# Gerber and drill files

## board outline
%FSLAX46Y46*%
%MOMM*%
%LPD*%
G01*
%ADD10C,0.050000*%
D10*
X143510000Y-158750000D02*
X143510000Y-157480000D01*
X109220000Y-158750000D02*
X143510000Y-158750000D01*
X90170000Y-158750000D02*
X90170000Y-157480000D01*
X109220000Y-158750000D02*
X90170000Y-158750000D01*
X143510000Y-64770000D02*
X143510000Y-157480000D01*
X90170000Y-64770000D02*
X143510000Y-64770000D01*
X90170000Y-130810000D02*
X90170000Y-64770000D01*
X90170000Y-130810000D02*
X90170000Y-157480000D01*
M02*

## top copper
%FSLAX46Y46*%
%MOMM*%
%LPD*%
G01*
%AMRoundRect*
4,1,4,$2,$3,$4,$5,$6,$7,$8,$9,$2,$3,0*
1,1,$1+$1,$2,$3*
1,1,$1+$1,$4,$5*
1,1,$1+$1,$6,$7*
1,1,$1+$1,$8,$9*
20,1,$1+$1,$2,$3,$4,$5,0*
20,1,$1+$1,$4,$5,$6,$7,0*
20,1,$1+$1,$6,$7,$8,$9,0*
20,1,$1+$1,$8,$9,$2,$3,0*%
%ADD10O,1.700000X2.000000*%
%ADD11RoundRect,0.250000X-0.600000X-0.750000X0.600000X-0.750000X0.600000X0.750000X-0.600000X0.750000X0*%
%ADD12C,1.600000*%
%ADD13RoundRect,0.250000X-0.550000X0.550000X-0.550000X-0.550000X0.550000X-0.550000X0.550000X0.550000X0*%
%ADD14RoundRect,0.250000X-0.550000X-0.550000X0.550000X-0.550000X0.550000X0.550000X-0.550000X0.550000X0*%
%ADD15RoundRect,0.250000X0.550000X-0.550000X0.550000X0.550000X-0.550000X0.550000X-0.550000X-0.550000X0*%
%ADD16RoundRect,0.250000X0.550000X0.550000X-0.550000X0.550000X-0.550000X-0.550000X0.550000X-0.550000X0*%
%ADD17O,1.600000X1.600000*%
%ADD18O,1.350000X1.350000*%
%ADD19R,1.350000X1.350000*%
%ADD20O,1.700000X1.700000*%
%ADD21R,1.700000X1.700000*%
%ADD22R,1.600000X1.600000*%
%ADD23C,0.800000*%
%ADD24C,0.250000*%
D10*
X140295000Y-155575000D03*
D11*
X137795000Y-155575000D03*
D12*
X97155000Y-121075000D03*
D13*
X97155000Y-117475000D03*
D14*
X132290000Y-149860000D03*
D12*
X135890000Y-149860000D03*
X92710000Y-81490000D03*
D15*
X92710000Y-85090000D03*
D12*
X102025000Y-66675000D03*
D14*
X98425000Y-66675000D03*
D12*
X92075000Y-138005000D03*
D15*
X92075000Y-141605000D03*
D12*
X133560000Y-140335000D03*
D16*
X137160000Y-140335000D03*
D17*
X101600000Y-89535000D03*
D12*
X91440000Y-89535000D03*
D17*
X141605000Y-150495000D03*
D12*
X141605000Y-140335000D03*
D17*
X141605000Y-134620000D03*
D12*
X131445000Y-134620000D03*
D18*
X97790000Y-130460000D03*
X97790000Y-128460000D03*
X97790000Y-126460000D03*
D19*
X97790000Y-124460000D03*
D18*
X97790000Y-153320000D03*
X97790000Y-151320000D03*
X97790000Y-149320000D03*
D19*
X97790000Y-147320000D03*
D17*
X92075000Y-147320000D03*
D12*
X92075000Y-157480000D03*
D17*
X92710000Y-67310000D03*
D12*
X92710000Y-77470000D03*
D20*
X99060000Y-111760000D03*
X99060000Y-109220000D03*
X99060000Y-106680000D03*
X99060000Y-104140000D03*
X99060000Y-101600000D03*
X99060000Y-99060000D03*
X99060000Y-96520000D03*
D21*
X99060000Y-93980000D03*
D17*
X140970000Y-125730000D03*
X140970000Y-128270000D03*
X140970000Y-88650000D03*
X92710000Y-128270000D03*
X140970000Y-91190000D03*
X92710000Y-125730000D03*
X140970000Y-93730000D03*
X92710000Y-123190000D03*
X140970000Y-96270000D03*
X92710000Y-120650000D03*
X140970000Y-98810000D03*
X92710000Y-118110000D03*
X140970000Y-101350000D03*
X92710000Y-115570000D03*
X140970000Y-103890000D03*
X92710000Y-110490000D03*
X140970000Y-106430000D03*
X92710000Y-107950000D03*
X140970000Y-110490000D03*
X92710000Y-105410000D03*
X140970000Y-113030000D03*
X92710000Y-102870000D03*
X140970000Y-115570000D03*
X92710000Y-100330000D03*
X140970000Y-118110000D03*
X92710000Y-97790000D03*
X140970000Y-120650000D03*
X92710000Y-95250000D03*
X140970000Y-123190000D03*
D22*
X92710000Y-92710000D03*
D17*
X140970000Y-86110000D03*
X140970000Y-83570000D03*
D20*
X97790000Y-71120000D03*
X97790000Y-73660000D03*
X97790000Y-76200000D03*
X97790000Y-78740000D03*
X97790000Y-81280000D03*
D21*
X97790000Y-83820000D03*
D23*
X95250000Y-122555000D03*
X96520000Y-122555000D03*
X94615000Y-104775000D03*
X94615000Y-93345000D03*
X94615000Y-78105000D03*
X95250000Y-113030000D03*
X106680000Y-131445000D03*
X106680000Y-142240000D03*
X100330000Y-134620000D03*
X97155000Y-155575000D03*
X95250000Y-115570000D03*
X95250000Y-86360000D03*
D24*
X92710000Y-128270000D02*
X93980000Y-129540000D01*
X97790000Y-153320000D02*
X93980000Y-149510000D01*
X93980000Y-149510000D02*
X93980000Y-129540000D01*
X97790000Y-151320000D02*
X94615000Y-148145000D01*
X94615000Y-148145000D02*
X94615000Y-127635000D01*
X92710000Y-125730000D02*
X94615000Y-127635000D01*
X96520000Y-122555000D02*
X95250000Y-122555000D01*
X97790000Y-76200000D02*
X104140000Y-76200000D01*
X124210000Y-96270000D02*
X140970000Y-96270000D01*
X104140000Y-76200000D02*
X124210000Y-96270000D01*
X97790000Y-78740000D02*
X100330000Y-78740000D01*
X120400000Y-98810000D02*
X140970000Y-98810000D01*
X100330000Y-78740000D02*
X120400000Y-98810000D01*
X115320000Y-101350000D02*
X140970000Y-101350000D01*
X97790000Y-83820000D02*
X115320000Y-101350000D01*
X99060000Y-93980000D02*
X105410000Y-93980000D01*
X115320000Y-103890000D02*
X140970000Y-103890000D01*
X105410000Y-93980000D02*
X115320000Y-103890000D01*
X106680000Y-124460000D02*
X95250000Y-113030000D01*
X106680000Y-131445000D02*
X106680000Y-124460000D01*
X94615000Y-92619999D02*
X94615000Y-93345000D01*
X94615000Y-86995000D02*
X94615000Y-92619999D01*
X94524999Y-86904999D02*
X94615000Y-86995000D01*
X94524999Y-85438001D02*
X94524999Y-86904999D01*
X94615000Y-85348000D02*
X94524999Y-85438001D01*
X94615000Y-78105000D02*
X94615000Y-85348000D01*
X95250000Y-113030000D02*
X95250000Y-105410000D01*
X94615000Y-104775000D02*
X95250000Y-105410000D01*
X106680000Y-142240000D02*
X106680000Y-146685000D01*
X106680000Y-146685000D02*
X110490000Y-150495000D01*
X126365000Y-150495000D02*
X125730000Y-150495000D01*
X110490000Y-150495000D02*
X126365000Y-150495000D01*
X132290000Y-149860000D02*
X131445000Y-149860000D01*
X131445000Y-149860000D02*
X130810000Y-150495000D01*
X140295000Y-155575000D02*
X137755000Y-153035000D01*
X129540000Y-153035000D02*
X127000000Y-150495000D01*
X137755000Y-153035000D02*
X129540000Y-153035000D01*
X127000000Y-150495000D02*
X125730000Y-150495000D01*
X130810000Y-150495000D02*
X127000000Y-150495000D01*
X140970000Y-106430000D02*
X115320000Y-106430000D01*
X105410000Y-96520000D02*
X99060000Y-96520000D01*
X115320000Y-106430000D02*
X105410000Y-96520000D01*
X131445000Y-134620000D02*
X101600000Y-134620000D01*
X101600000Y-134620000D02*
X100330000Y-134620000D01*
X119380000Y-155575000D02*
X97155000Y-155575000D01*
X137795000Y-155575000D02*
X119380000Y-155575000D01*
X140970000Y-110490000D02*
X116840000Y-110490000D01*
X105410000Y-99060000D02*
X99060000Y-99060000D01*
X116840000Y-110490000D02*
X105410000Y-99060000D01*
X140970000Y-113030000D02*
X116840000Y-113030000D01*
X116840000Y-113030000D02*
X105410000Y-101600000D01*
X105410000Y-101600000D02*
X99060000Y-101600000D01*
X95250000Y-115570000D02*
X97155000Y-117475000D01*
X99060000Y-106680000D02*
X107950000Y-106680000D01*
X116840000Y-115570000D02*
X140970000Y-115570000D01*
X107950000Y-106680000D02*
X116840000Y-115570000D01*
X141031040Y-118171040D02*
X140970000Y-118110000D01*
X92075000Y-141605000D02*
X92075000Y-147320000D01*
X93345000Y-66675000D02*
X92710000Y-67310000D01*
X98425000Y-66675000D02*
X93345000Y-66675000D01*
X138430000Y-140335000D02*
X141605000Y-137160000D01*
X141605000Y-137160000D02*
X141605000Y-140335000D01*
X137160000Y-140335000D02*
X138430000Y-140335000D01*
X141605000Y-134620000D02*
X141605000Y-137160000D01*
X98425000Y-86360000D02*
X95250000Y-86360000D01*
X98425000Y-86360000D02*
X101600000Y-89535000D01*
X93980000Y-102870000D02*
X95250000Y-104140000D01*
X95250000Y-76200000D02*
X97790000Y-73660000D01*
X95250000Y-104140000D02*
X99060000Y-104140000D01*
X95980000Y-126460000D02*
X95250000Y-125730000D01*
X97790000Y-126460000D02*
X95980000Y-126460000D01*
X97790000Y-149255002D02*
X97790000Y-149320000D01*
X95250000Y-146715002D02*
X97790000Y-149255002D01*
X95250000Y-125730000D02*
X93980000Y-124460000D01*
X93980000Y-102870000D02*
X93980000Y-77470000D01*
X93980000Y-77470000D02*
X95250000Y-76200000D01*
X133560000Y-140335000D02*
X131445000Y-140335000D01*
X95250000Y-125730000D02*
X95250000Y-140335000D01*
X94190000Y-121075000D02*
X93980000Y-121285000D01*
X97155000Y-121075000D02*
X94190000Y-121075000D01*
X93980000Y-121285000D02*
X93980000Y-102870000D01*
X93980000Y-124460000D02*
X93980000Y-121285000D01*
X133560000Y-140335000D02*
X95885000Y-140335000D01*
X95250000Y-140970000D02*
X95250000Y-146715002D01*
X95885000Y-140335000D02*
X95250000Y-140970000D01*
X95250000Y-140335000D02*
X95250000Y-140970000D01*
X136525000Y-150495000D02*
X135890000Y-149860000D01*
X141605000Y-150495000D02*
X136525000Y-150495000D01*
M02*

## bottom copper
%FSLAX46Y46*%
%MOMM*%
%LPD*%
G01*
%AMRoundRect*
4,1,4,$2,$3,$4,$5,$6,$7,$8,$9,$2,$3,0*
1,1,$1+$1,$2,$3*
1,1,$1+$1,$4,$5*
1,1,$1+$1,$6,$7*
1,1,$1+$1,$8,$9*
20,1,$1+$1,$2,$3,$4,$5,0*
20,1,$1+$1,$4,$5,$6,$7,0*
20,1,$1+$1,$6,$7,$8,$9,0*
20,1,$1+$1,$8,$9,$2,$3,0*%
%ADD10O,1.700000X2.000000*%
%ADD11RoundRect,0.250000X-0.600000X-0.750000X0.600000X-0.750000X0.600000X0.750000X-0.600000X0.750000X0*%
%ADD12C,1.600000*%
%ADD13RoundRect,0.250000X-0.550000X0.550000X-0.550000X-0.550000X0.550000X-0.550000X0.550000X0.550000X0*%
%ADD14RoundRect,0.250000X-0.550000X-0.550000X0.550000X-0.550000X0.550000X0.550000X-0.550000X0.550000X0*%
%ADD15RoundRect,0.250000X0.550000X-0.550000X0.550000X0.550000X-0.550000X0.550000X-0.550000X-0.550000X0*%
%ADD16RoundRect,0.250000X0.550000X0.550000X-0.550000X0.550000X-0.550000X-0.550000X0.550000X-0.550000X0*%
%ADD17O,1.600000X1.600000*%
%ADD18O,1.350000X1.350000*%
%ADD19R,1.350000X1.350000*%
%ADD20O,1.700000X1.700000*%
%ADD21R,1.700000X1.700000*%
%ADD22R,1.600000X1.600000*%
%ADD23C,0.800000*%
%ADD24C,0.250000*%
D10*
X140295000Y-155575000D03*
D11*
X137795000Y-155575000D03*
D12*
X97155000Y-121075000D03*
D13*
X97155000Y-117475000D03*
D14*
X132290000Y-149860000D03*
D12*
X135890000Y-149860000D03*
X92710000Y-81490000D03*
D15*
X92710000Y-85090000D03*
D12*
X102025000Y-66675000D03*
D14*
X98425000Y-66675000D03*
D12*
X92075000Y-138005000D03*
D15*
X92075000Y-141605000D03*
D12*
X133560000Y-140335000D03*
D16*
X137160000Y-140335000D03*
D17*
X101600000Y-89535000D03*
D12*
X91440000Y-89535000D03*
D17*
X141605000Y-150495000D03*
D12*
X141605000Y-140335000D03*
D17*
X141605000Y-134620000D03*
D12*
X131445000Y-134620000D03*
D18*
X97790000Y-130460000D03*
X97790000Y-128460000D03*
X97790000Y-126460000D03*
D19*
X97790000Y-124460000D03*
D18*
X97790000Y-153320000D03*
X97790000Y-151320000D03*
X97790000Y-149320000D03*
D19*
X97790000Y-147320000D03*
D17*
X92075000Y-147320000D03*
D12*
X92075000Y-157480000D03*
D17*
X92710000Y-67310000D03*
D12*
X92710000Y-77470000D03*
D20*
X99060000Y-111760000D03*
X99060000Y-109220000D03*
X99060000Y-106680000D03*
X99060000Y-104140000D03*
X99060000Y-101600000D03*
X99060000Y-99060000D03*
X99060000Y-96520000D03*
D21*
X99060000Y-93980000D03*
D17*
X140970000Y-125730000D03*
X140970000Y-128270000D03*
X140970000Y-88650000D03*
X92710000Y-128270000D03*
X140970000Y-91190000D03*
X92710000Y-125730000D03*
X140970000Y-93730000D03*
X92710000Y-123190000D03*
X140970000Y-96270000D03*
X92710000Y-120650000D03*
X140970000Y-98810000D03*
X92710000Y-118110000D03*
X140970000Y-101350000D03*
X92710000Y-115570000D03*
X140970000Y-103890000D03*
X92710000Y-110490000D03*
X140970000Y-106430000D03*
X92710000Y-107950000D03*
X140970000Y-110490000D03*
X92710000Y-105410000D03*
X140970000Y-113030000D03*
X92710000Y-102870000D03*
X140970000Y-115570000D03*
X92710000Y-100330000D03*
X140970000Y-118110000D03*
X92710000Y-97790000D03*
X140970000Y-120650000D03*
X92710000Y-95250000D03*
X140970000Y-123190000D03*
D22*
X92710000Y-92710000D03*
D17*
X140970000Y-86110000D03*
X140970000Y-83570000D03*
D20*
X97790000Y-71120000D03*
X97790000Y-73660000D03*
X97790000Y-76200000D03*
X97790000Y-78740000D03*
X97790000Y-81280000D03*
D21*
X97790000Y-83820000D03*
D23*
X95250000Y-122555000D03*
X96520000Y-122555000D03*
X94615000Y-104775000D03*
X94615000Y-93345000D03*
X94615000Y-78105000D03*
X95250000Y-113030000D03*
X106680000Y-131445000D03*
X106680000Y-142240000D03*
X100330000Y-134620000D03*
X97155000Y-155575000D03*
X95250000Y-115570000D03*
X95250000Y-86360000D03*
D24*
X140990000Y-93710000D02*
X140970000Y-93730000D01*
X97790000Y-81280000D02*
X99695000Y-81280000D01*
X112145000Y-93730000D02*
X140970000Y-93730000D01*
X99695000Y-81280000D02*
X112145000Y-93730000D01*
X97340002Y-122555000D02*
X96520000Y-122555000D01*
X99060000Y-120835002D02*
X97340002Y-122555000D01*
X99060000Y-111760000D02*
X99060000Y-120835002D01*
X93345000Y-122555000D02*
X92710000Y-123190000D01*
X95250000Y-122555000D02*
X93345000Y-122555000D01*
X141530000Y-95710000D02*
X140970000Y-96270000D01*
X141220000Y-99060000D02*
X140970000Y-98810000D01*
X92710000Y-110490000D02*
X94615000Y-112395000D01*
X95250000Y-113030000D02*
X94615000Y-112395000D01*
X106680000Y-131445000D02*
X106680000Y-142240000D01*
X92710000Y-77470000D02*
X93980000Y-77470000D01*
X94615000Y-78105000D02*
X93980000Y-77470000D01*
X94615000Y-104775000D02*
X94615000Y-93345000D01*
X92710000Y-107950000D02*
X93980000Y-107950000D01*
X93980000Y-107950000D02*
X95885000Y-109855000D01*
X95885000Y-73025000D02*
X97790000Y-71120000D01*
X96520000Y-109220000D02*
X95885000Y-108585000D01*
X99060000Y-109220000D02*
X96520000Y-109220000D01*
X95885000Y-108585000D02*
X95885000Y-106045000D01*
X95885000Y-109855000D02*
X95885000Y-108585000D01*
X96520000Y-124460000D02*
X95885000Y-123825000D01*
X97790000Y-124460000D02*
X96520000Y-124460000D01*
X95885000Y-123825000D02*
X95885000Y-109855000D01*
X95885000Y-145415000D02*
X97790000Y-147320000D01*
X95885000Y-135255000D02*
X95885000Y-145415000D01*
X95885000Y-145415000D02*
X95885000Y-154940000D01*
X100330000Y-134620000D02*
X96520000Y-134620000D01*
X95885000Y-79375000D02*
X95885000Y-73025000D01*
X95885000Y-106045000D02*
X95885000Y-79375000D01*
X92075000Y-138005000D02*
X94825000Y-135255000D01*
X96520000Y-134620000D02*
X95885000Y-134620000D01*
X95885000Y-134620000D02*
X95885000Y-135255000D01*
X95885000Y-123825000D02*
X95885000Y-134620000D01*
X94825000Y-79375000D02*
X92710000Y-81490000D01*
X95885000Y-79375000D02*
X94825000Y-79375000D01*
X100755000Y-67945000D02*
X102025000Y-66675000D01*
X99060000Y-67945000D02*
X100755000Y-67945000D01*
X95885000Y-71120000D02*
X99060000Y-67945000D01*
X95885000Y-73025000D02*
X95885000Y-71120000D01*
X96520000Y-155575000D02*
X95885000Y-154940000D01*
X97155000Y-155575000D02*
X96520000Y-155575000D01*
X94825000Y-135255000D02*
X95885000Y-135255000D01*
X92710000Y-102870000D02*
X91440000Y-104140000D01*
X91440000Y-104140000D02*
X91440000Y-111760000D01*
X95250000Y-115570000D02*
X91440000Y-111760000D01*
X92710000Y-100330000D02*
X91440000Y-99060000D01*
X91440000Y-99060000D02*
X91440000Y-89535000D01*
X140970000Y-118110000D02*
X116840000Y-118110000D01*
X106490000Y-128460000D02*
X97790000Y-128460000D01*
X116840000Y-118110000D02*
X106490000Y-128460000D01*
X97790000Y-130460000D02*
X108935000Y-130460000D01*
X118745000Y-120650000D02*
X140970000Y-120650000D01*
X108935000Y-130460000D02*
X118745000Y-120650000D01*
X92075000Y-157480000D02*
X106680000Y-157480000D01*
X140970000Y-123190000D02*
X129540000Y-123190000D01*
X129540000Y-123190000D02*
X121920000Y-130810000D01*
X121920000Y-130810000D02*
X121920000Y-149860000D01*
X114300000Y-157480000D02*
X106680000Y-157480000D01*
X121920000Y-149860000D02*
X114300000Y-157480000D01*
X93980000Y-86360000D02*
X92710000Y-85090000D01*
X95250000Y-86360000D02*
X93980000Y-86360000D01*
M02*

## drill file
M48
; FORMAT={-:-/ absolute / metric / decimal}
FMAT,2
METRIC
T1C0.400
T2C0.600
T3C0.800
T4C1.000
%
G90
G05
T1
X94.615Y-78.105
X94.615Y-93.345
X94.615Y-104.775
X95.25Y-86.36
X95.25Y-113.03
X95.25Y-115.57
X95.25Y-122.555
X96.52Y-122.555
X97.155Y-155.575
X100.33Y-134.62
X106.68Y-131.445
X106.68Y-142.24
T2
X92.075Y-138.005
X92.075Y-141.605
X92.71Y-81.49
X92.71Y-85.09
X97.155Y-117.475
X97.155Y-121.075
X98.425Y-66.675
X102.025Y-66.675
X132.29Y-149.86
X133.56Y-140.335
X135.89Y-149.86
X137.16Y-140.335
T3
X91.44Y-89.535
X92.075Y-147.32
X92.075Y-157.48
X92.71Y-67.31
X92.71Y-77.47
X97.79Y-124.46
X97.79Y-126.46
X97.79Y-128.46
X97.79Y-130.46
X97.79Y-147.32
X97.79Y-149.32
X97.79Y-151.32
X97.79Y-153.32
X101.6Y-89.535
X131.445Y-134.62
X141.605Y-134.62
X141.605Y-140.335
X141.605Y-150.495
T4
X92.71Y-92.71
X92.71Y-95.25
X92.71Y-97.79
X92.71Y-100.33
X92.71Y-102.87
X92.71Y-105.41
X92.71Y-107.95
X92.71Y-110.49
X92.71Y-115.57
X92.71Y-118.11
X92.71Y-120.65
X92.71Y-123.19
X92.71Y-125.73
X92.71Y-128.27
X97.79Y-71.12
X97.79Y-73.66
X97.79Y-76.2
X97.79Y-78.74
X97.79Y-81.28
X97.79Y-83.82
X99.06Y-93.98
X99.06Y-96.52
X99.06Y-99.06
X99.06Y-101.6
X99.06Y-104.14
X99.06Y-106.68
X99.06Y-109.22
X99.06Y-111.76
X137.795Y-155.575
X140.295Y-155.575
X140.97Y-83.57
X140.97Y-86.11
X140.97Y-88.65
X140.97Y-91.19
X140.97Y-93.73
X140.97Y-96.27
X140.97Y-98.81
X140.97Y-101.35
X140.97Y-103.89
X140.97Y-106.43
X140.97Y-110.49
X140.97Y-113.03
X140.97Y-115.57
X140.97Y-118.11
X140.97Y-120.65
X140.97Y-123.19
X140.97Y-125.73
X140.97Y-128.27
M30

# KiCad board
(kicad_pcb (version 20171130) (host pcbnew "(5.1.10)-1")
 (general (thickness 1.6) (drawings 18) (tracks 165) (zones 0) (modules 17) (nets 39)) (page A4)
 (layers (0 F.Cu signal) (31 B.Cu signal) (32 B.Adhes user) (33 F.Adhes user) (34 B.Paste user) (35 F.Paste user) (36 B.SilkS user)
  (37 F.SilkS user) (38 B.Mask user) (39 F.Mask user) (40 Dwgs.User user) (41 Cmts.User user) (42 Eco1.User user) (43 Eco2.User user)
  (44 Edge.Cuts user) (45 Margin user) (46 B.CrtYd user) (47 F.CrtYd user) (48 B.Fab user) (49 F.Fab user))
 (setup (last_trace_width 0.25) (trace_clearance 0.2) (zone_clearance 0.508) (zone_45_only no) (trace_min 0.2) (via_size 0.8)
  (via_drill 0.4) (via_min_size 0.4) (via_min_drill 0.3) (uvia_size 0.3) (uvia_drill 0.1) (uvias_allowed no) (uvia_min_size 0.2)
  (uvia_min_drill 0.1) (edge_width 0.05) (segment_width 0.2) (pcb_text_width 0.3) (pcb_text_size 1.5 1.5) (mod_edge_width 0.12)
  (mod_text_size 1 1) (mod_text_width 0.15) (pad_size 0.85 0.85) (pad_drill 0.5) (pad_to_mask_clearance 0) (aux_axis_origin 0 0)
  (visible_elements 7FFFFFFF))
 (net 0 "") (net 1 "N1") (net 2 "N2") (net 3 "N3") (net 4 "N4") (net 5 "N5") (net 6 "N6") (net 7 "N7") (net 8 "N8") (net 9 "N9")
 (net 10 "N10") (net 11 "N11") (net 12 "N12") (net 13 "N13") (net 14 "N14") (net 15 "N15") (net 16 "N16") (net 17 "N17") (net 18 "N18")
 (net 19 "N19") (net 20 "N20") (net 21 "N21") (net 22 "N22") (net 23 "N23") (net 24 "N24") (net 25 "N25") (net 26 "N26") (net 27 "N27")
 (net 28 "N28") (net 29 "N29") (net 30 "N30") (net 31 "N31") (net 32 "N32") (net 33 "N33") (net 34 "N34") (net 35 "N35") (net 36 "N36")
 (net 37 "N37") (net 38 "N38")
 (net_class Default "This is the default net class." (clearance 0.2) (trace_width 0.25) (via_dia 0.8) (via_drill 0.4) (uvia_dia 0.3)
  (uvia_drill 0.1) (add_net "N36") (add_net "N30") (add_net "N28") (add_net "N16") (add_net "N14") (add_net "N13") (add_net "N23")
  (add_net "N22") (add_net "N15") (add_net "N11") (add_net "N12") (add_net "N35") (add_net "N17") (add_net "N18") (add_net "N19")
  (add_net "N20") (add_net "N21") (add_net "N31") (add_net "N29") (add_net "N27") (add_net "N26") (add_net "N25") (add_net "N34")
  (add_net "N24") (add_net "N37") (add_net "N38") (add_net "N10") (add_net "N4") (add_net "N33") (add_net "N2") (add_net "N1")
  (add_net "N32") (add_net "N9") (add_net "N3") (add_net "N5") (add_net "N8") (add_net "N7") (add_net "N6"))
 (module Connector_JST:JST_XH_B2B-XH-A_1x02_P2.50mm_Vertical (layer B.Cu) (at 137.795 155.575)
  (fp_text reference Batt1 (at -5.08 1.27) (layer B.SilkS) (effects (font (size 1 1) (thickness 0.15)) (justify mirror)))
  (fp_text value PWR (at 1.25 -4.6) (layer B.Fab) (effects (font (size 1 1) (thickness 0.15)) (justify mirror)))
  (pad 2 thru_hole oval (at 2.5 0) (size 1.7 2) (drill 1) (layers *.Cu *.Mask) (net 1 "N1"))
  (pad 1 thru_hole roundrect (at 0 0) (size 1.7 2) (drill 1) (layers *.Cu *.Mask) (roundrect_rratio 0.1470588235294118) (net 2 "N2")))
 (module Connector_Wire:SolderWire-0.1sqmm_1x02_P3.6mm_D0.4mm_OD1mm (layer F.Cu) (at 97.155 117.475 270)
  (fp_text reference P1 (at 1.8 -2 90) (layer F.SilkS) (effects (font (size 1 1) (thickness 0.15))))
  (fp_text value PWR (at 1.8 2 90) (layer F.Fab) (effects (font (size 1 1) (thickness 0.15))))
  (pad 2 thru_hole circle (at 3.6 0 270) (size 1.6 1.6) (drill 0.6) (layers *.Cu *.Mask) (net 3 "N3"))
  (pad 1 thru_hole roundrect (at 0 0 270) (size 1.6 1.6) (drill 0.6) (layers *.Cu *.Mask) (roundrect_rratio 0.15625) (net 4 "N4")))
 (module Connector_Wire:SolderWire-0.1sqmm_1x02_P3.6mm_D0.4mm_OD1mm (layer F.Cu) (at 132.29 149.86)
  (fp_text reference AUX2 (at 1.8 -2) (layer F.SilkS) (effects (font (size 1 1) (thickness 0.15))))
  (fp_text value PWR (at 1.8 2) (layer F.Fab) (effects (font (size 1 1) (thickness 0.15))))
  (pad 1 thru_hole roundrect (at 0 0) (size 1.6 1.6) (drill 0.6) (layers *.Cu *.Mask) (roundrect_rratio 0.15625) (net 1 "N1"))
  (pad 2 thru_hole circle (at 3.6 0) (size 1.6 1.6) (drill 0.6) (layers *.Cu *.Mask) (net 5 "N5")))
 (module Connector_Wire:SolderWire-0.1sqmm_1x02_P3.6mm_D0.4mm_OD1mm (layer F.Cu) (at 92.71 85.09 90)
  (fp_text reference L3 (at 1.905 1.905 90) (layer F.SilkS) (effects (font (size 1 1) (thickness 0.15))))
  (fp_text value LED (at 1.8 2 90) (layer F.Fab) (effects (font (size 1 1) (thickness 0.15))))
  (pad 2 thru_hole circle (at 3.6 0 90) (size 1.6 1.6) (drill 0.6) (layers *.Cu *.Mask) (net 2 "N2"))
  (pad 1 thru_hole roundrect (at 0 0 90) (size 1.6 1.6) (drill 0.6) (layers *.Cu *.Mask) (roundrect_rratio 0.15625) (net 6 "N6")))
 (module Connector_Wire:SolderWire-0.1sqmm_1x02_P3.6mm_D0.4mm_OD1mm (layer F.Cu) (at 98.425 66.675)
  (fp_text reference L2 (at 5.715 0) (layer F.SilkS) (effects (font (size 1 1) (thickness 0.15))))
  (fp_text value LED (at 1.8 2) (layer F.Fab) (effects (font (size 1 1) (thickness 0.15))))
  (pad 2 thru_hole circle (at 3.6 0) (size 1.6 1.6) (drill 0.6) (layers *.Cu *.Mask) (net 2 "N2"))
  (pad 1 thru_hole roundrect (at 0 0) (size 1.6 1.6) (drill 0.6) (layers *.Cu *.Mask) (roundrect_rratio 0.15625) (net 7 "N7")))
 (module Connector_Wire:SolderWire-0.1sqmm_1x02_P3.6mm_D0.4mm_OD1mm (layer F.Cu) (at 92.075 141.605 90)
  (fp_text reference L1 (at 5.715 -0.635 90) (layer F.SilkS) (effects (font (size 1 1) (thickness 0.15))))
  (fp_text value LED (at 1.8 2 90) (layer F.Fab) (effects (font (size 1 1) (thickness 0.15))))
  (pad 2 thru_hole circle (at 3.6 0 90) (size 1.6 1.6) (drill 0.6) (layers *.Cu *.Mask) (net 2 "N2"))
  (pad 1 thru_hole roundrect (at 0 0 90) (size 1.6 1.6) (drill 0.6) (layers *.Cu *.Mask) (roundrect_rratio 0.15625) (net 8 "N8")))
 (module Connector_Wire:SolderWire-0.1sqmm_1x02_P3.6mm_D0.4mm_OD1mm (layer F.Cu) (at 137.16 140.335 180)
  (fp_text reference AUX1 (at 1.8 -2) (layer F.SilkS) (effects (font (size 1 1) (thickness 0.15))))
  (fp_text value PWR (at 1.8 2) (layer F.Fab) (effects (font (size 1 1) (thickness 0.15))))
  (pad 2 thru_hole circle (at 3.6 0 180) (size 1.6 1.6) (drill 0.6) (layers *.Cu *.Mask) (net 3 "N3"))
  (pad 1 thru_hole roundrect (at 0 0 180) (size 1.6 1.6) (drill 0.6) (layers *.Cu *.Mask) (roundrect_rratio 0.15625) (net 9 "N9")))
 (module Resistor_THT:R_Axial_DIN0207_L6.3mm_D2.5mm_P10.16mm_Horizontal (layer F.Cu) (at 91.44 89.535)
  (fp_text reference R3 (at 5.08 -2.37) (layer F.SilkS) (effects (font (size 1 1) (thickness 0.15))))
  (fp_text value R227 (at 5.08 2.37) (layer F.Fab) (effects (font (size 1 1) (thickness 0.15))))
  (pad 2 thru_hole oval (at 10.16 0) (size 1.6 1.6) (drill 0.8) (layers *.Cu *.Mask) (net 6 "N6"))
  (pad 1 thru_hole circle (at 0 0) (size 1.6 1.6) (drill 0.8) (layers *.Cu *.Mask) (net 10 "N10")))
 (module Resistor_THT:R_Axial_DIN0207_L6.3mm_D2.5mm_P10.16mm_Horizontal (layer B.Cu) (at 141.605 140.335 270)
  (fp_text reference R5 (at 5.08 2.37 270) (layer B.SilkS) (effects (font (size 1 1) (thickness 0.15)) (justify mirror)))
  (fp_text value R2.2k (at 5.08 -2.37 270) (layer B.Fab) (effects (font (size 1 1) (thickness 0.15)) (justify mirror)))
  (pad 2 thru_hole oval (at 10.16 0 270) (size 1.6 1.6) (drill 0.8) (layers *.Cu *.Mask) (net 5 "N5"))
  (pad 1 thru_hole circle (at 0 0 270) (size 1.6 1.6) (drill 0.8) (layers *.Cu *.Mask) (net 9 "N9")))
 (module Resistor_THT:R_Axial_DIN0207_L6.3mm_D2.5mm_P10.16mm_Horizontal (layer B.Cu) (at 131.445 134.62)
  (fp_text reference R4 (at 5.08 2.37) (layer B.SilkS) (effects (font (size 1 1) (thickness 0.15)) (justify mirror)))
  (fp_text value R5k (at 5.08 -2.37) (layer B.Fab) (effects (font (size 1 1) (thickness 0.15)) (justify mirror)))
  (pad 2 thru_hole oval (at 10.16 0) (size 1.6 1.6) (drill 0.8) (layers *.Cu *.Mask) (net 9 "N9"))
  (pad 1 thru_hole circle (at 0 0) (size 1.6 1.6) (drill 0.8) (layers *.Cu *.Mask) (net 2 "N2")))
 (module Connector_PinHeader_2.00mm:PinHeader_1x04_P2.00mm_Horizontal (layer F.Cu) (at 97.79 124.46)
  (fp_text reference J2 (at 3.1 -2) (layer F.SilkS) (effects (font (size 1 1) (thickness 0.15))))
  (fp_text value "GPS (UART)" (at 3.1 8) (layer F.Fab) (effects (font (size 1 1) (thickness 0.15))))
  (pad 4 thru_hole oval (at 0 6) (size 1.35 1.35) (drill 0.8) (layers *.Cu *.Mask) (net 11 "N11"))
  (pad 3 thru_hole oval (at 0 4) (size 1.35 1.35) (drill 0.8) (layers *.Cu *.Mask) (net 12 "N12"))
  (pad 2 thru_hole oval (at 0 2) (size 1.35 1.35) (drill 0.8) (layers *.Cu *.Mask) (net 3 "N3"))
  (pad 1 thru_hole rect (at 0 0) (size 1.35 1.35) (drill 0.8) (layers *.Cu *.Mask) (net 2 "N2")))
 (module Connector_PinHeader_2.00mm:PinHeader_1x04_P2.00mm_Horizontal (layer F.Cu) (at 97.79 147.32)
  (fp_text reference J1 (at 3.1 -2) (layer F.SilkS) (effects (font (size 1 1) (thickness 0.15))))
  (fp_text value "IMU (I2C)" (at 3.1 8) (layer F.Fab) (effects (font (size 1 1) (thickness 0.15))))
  (pad 4 thru_hole oval (at 0 6) (size 1.35 1.35) (drill 0.8) (layers *.Cu *.Mask) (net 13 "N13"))
  (pad 3 thru_hole oval (at 0 4) (size 1.35 1.35) (drill 0.8) (layers *.Cu *.Mask) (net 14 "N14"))
  (pad 2 thru_hole oval (at 0 2) (size 1.35 1.35) (drill 0.8) (layers *.Cu *.Mask) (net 3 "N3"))
  (pad 1 thru_hole rect (at 0 0) (size 1.35 1.35) (drill 0.8) (layers *.Cu *.Mask) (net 2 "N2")))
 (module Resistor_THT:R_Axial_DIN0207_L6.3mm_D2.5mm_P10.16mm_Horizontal (layer B.Cu) (at 92.075 157.48 90)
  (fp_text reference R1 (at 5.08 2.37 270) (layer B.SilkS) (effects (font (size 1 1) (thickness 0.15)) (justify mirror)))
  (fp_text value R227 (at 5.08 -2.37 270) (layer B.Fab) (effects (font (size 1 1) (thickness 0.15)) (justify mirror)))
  (pad 2 thru_hole oval (at 10.16 0 90) (size 1.6 1.6) (drill 0.8) (layers *.Cu *.Mask) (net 8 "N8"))
  (pad 1 thru_hole circle (at 0 0 90) (size 1.6 1.6) (drill 0.8) (layers *.Cu *.Mask) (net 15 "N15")))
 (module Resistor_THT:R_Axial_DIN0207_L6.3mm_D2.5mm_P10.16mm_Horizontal (layer F.Cu) (at 92.71 77.47 90)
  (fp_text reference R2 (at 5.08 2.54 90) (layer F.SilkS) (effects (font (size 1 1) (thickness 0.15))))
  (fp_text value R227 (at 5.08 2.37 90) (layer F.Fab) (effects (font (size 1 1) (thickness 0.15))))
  (pad 2 thru_hole oval (at 10.16 0 90) (size 1.6 1.6) (drill 0.8) (layers *.Cu *.Mask) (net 7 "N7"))
  (pad 1 thru_hole circle (at 0 0 90) (size 1.6 1.6) (drill 0.8) (layers *.Cu *.Mask) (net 1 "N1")))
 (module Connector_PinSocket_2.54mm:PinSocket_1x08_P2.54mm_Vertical (layer F.Cu) (at 99.06 93.98)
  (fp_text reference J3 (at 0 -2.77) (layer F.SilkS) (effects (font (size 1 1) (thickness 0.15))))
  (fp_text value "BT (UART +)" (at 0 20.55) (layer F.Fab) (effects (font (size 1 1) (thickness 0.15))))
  (pad 8 thru_hole oval (at 0 17.78) (size 1.7 1.7) (drill 1) (layers *.Cu *.Mask) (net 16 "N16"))
  (pad 7 thru_hole oval (at 0 15.24) (size 1.7 1.7) (drill 1) (layers *.Cu *.Mask) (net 2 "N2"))
  (pad 6 thru_hole oval (at 0 12.7) (size 1.7 1.7) (drill 1) (layers *.Cu *.Mask) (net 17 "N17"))
  (pad 5 thru_hole oval (at 0 10.16) (size 1.7 1.7) (drill 1) (layers *.Cu *.Mask) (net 3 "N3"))
  (pad 4 thru_hole oval (at 0 7.62) (size 1.7 1.7) (drill 1) (layers *.Cu *.Mask) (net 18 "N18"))
  (pad 3 thru_hole oval (at 0 5.08) (size 1.7 1.7) (drill 1) (layers *.Cu *.Mask) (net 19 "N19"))
  (pad 2 thru_hole oval (at 0 2.54) (size 1.7 1.7) (drill 1) (layers *.Cu *.Mask) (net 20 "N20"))
  (pad 1 thru_hole rect (at 0 0) (size 1.7 1.7) (drill 1) (layers *.Cu *.Mask) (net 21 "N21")))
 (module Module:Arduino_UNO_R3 (layer B.Cu) (at 92.71 92.71 270)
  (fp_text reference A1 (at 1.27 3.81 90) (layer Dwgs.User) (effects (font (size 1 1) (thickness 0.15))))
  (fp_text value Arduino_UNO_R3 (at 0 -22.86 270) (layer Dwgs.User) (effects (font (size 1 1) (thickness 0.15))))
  (pad 16 thru_hole oval (at 33.02 -48.26 180) (size 1.6 1.6) (drill 1) (layers *.Cu *.Mask) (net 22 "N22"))
  (pad 15 thru_hole oval (at 35.56 -48.26 180) (size 1.6 1.6) (drill 1) (layers *.Cu *.Mask) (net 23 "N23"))
  (pad 30 thru_hole oval (at -4.06 -48.26 180) (size 1.6 1.6) (drill 1) (layers *.Cu *.Mask) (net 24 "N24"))
  (pad 14 thru_hole oval (at 35.56 0 180) (size 1.6 1.6) (drill 1) (layers *.Cu *.Mask) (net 13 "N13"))
  (pad 29 thru_hole oval (at -1.52 -48.26 180) (size 1.6 1.6) (drill 1) (layers *.Cu *.Mask) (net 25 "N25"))
  (pad 13 thru_hole oval (at 33.02 0 180) (size 1.6 1.6) (drill 1) (layers *.Cu *.Mask) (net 14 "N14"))
  (pad 28 thru_hole oval (at 1.02 -48.26 180) (size 1.6 1.6) (drill 1) (layers *.Cu *.Mask) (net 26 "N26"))
  (pad 12 thru_hole oval (at 30.48 0 180) (size 1.6 1.6) (drill 1) (layers *.Cu *.Mask) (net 16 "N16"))
  (pad 27 thru_hole oval (at 3.56 -48.26 180) (size 1.6 1.6) (drill 1) (layers *.Cu *.Mask) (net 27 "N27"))
  (pad 11 thru_hole oval (at 27.94 0 180) (size 1.6 1.6) (drill 1) (layers *.Cu *.Mask) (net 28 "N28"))
  (pad 26 thru_hole oval (at 6.1 -48.26 180) (size 1.6 1.6) (drill 1) (layers *.Cu *.Mask) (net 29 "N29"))
  (pad 10 thru_hole oval (at 25.4 0 180) (size 1.6 1.6) (drill 1) (layers *.Cu *.Mask) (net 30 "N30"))
  (pad 25 thru_hole oval (at 8.64 -48.26 180) (size 1.6 1.6) (drill 1) (layers *.Cu *.Mask) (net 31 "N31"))
  (pad 9 thru_hole oval (at 22.86 0 180) (size 1.6 1.6) (drill 1) (layers *.Cu *.Mask) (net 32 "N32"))
  (pad 24 thru_hole oval (at 11.18 -48.26 180) (size 1.6 1.6) (drill 1) (layers *.Cu *.Mask) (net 21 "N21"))
  (pad 8 thru_hole oval (at 17.78 0 180) (size 1.6 1.6) (drill 1) (layers *.Cu *.Mask) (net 1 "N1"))
  (pad 23 thru_hole oval (at 13.72 -48.26 180) (size 1.6 1.6) (drill 1) (layers *.Cu *.Mask) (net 20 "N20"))
  (pad 7 thru_hole oval (at 15.24 0 180) (size 1.6 1.6) (drill 1) (layers *.Cu *.Mask) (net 2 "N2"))
  (pad 22 thru_hole oval (at 17.78 -48.26 180) (size 1.6 1.6) (drill 1) (layers *.Cu *.Mask) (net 19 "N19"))
  (pad 6 thru_hole oval (at 12.7 0 180) (size 1.6 1.6) (drill 1) (layers *.Cu *.Mask) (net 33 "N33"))
  (pad 21 thru_hole oval (at 20.32 -48.26 180) (size 1.6 1.6) (drill 1) (layers *.Cu *.Mask) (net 18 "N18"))
  (pad 5 thru_hole oval (at 10.16 0 180) (size 1.6 1.6) (drill 1) (layers *.Cu *.Mask) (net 4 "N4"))
  (pad 20 thru_hole oval (at 22.86 -48.26 180) (size 1.6 1.6) (drill 1) (layers *.Cu *.Mask) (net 17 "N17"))
  (pad 4 thru_hole oval (at 7.62 0 180) (size 1.6 1.6) (drill 1) (layers *.Cu *.Mask) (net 10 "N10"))
  (pad 19 thru_hole oval (at 25.4 -48.26 180) (size 1.6 1.6) (drill 1) (layers *.Cu *.Mask) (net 12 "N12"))
  (pad 3 thru_hole oval (at 5.08 0 180) (size 1.6 1.6) (drill 1) (layers *.Cu *.Mask) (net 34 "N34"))
  (pad 18 thru_hole oval (at 27.94 -48.26 180) (size 1.6 1.6) (drill 1) (layers *.Cu *.Mask) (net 11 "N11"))
  (pad 2 thru_hole oval (at 2.54 0 180) (size 1.6 1.6) (drill 1) (layers *.Cu *.Mask) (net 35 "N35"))
  (pad 17 thru_hole oval (at 30.48 -48.26 180) (size 1.6 1.6) (drill 1) (layers *.Cu *.Mask) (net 15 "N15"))
  (pad 1 thru_hole rect (at 0 0 180) (size 1.6 1.6) (drill 1) (layers *.Cu *.Mask) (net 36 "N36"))
  (pad 31 thru_hole oval (at -6.6 -48.26 180) (size 1.6 1.6) (drill 1) (layers *.Cu *.Mask) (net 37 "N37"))
  (pad 32 thru_hole oval (at -9.14 -48.26 180) (size 1.6 1.6) (drill 1) (layers *.Cu *.Mask) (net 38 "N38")))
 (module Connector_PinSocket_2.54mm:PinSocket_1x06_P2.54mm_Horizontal (layer F.Cu) (at 97.79 83.82 180)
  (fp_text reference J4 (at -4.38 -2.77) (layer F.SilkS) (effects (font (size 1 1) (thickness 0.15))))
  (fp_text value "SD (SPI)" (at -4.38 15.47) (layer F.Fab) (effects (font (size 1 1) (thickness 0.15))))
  (pad 6 thru_hole oval (at 0 12.7 180) (size 1.7 1.7) (drill 1) (layers *.Cu *.Mask) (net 2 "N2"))
  (pad 5 thru_hole oval (at 0 10.16 180) (size 1.7 1.7) (drill 1) (layers *.Cu *.Mask) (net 3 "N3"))
  (pad 4 thru_hole oval (at 0 7.62 180) (size 1.7 1.7) (drill 1) (layers *.Cu *.Mask) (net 27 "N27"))
  (pad 3 thru_hole oval (at 0 5.08 180) (size 1.7 1.7) (drill 1) (layers *.Cu *.Mask) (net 29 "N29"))
  (pad 2 thru_hole oval (at 0 2.54 180) (size 1.7 1.7) (drill 1) (layers *.Cu *.Mask) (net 26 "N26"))
  (pad 1 thru_hole rect (at 0 0 180) (size 1.7 1.7) (drill 1) (layers *.Cu *.Mask) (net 31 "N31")))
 (gr_line (start 143.51 158.75) (end 143.51 157.48) (layer Edge.Cuts) (width 0.05))
 (gr_line (start 109.22 158.75) (end 143.51 158.75) (layer Edge.Cuts) (width 0.05))
 (gr_line (start 90.17 158.75) (end 90.17 157.48) (layer Edge.Cuts) (width 0.05))
 (gr_line (start 109.22 158.75) (end 90.17 158.75) (layer Edge.Cuts) (width 0.05))
 (gr_line (start 143.51 64.77) (end 143.51 157.48) (layer Edge.Cuts) (width 0.05))
 (gr_line (start 90.17 64.77) (end 143.51 64.77) (layer Edge.Cuts) (width 0.05))
 (gr_line (start 90.17 130.81) (end 90.17 64.77) (layer Edge.Cuts) (width 0.05))
 (gr_line (start 90.17 130.81) (end 90.17 157.48) (layer Edge.Cuts) (width 0.05))
 (segment (start 92.71 128.27) (end 93.98 129.54) (width 0.25) (layer F.Cu) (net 13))
 (segment (start 97.79 153.32) (end 93.98 149.51) (width 0.25) (layer F.Cu) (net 13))
 (segment (start 93.98 149.51) (end 93.98 129.54) (width 0.25) (layer F.Cu) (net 13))
 (segment (start 97.79 151.32) (end 94.615 148.145) (width 0.25) (layer F.Cu) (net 14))
 (segment (start 94.615 148.145) (end 94.615 127.635) (width 0.25) (layer F.Cu) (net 14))
 (segment (start 92.71 125.73) (end 94.615 127.635) (width 0.25) (layer F.Cu) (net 14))
 (segment (start 140.99 93.71) (end 140.97 93.73) (width 0.25) (layer B.Cu) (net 26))
 (segment (start 97.79 81.28) (end 99.695 81.28) (width 0.25) (layer B.Cu) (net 26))
 (segment (start 112.145 93.73) (end 140.97 93.73) (width 0.25) (layer B.Cu) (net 26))
 (segment (start 99.695 81.28) (end 112.145 93.73) (width 0.25) (layer B.Cu) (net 26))
 (via (at 95.25 122.555) (size 0.8) (drill 0.4) (layers F.Cu B.Cu) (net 16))
 (via (at 96.52 122.555) (size 0.8) (drill 0.4) (layers F.Cu B.Cu) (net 16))
 (segment (start 97.340002 122.555) (end 96.52 122.555) (width 0.25) (layer B.Cu) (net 16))
 (segment (start 99.06 120.835002) (end 97.340002 122.555) (width 0.25) (layer B.Cu) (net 16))
 (segment (start 99.06 111.76) (end 99.06 120.835002) (width 0.25) (layer B.Cu) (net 16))
 (segment (start 96.52 122.555) (end 95.25 122.555) (width 0.25) (layer F.Cu) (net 16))
 (segment (start 93.345 122.555) (end 92.71 123.19) (width 0.25) (layer B.Cu) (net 16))
 (segment (start 95.25 122.555) (end 93.345 122.555) (width 0.25) (layer B.Cu) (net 16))
 (segment (start 141.53 95.71) (end 140.97 96.27) (width 0.25) (layer B.Cu) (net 27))
 (segment (start 97.79 76.2) (end 104.14 76.2) (width 0.25) (layer F.Cu) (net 27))
 (segment (start 124.21 96.27) (end 140.97 96.27) (width 0.25) (layer F.Cu) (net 27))
 (segment (start 104.14 76.2) (end 124.21 96.27) (width 0.25) (layer F.Cu) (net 27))
 (segment (start 141.22 99.06) (end 140.97 98.81) (width 0.25) (layer B.Cu) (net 29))
 (segment (start 97.79 78.74) (end 100.33 78.74) (width 0.25) (layer F.Cu) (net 29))
 (segment (start 120.4 98.81) (end 140.97 98.81) (width 0.25) (layer F.Cu) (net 29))
 (segment (start 100.33 78.74) (end 120.4 98.81) (width 0.25) (layer F.Cu) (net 29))
 (segment (start 115.32 101.35) (end 140.97 101.35) (width 0.25) (layer F.Cu) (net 31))
 (segment (start 97.79 83.82) (end 115.32 101.35) (width 0.25) (layer F.Cu) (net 31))
 (segment (start 99.06 93.98) (end 105.41 93.98) (width 0.25) (layer F.Cu) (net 21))
 (segment (start 115.32 103.89) (end 140.97 103.89) (width 0.25) (layer F.Cu) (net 21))
 (segment (start 105.41 93.98) (end 115.32 103.89) (width 0.25) (layer F.Cu) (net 21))
 (via (at 94.615 104.775) (size 0.8) (drill 0.4) (layers F.Cu B.Cu) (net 1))
 (via (at 94.615 93.345) (size 0.8) (drill 0.4) (layers F.Cu B.Cu) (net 1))
 (via (at 94.615 78.105) (size 0.8) (drill 0.4) (layers F.Cu B.Cu) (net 1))
 (via (at 95.25 113.03) (size 0.8) (drill 0.4) (layers F.Cu B.Cu) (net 1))
 (segment (start 92.71 110.49) (end 94.615 112.395) (width 0.25) (layer B.Cu) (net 1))
 (segment (start 95.25 113.03) (end 94.615 112.395) (width 0.25) (layer B.Cu) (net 1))
 (segment (start 106.68 124.46) (end 95.25 113.03) (width 0.25) (layer F.Cu) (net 1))
 (segment (start 106.68 131.445) (end 106.68 124.46) (width 0.25) (layer F.Cu) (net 1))
 (segment (start 106.68 131.445) (end 106.68 142.24) (width 0.25) (layer B.Cu) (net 1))
 (segment (start 92.71 77.47) (end 93.98 77.47) (width 0.25) (layer B.Cu) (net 1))
 (segment (start 94.615 78.105) (end 93.98 77.47) (width 0.25) (layer B.Cu) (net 1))
 (segment (start 94.615 92.619999) (end 94.615 93.345) (width 0.25) (layer F.Cu) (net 1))
 (segment (start 94.615 86.995) (end 94.615 92.619999) (width 0.25) (layer F.Cu) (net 1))
 (segment (start 94.524999 86.904999) (end 94.615 86.995) (width 0.25) (layer F.Cu) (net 1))
 (segment (start 94.524999 85.438001) (end 94.524999 86.904999) (width 0.25) (layer F.Cu) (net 1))
 (segment (start 94.615 85.348) (end 94.524999 85.438001) (width 0.25) (layer F.Cu) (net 1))
 (segment (start 94.615 78.105) (end 94.615 85.348) (width 0.25) (layer F.Cu) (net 1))
 (segment (start 95.25 113.03) (end 95.25 105.41) (width 0.25) (layer F.Cu) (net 1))
 (segment (start 94.615 104.775) (end 95.25 105.41) (width 0.25) (layer F.Cu) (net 1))
 (segment (start 94.615 104.775) (end 94.615 93.345) (width 0.25) (layer B.Cu) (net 1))
 (segment (start 106.68 142.24) (end 106.68 146.685) (width 0.25) (layer F.Cu) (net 1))
 (segment (start 106.68 146.685) (end 110.49 150.495) (width 0.25) (layer F.Cu) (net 1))
 (segment (start 126.365 150.495) (end 125.73 150.495) (width 0.25) (layer F.Cu) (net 1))
 (segment (start 110.49 150.495) (end 126.365 150.495) (width 0.25) (layer F.Cu) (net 1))
 (via (at 106.68 131.445) (size 0.8) (drill 0.4) (layers F.Cu B.Cu) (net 1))
 (via (at 106.68 142.24) (size 0.8) (drill 0.4) (layers F.Cu B.Cu) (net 1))
 (segment (start 132.29 149.86) (end 131.445 149.86) (width 0.25) (layer F.Cu) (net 1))
 (segment (start 131.445 149.86) (end 130.81 150.495) (width 0.25) (layer F.Cu) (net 1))
 (segment (start 140.295 155.575) (end 137.755 153.035) (width 0.25) (layer F.Cu) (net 1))
 (segment (start 129.54 153.035) (end 127 150.495) (width 0.25) (layer F.Cu) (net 1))
 (segment (start 137.755 153.035) (end 129.54 153.035) (width 0.25) (layer F.Cu) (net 1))
 (segment (start 127 150.495) (end 125.73 150.495) (width 0.25) (layer F.Cu) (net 1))
 (segment (start 130.81 150.495) (end 127 150.495) (width 0.25) (layer F.Cu) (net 1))
 (segment (start 140.97 106.43) (end 115.32 106.43) (width 0.25) (layer F.Cu) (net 20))
 (segment (start 105.41 96.52) (end 99.06 96.52) (width 0.25) (layer F.Cu) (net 20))
 (segment (start 115.32 106.43) (end 105.41 96.52) (width 0.25) (layer F.Cu) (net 20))
 (via (at 100.33 134.62) (size 0.8) (drill 0.4) (layers F.Cu B.Cu) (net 2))
 (via (at 97.155 155.575) (size 0.8) (drill 0.4) (layers F.Cu B.Cu) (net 2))
 (segment (start 92.71 107.95) (end 93.98 107.95) (width 0.25) (layer B.Cu) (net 2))
 (segment (start 93.98 107.95) (end 95.885 109.855) (width 0.25) (layer B.Cu) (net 2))
 (segment (start 95.885 73.025) (end 97.79 71.12) (width 0.25) (layer B.Cu) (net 2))
 (segment (start 96.52 109.22) (end 95.885 108.585) (width 0.25) (layer B.Cu) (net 2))
 (segment (start 99.06 109.22) (end 96.52 109.22) (width 0.25) (layer B.Cu) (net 2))
 (segment (start 95.885 108.585) (end 95.885 106.045) (width 0.25) (layer B.Cu) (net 2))
 (segment (start 95.885 109.855) (end 95.885 108.585) (width 0.25) (layer B.Cu) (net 2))
 (segment (start 96.52 124.46) (end 95.885 123.825) (width 0.25) (layer B.Cu) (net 2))
 (segment (start 97.79 124.46) (end 96.52 124.46) (width 0.25) (layer B.Cu) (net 2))
 (segment (start 95.885 123.825) (end 95.885 109.855) (width 0.25) (layer B.Cu) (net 2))
 (segment (start 95.885 145.415) (end 97.79 147.32) (width 0.25) (layer B.Cu) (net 2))
 (segment (start 95.885 135.255) (end 95.885 145.415) (width 0.25) (layer B.Cu) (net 2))
 (segment (start 95.885 145.415) (end 95.885 154.94) (width 0.25) (layer B.Cu) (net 2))
 (segment (start 131.445 134.62) (end 101.6 134.62) (width 0.25) (layer F.Cu) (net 2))
 (segment (start 100.33 134.62) (end 96.52 134.62) (width 0.25) (layer B.Cu) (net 2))
 (segment (start 101.6 134.62) (end 100.33 134.62) (width 0.25) (layer F.Cu) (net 2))
 (segment (start 95.885 79.375) (end 95.885 73.025) (width 0.25) (layer B.Cu) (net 2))
 (segment (start 95.885 106.045) (end 95.885 79.375) (width 0.25) (layer B.Cu) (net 2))
 (segment (start 92.075 138.005) (end 94.825 135.255) (width 0.25) (layer B.Cu) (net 2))
 (segment (start 96.52 134.62) (end 95.885 134.62) (width 0.25) (layer B.Cu) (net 2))
 (segment (start 95.885 134.62) (end 95.885 135.255) (width 0.25) (layer B.Cu) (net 2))
 (segment (start 95.885 123.825) (end 95.885 134.62) (width 0.25) (layer B.Cu) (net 2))
 (segment (start 94.825 79.375) (end 92.71 81.49) (width 0.25) (layer B.Cu) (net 2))
 (segment (start 95.885 79.375) (end 94.825 79.375) (width 0.25) (layer B.Cu) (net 2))
 (segment (start 100.755 67.945) (end 102.025 66.675) (width 0.25) (layer B.Cu) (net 2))
 (segment (start 99.06 67.945) (end 100.755 67.945) (width 0.25) (layer B.Cu) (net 2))
 (segment (start 95.885 71.12) (end 99.06 67.945) (width 0.25) (layer B.Cu) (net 2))
 (segment (start 95.885 73.025) (end 95.885 71.12) (width 0.25) (layer B.Cu) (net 2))
 (segment (start 119.38 155.575) (end 97.155 155.575) (width 0.25) (layer F.Cu) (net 2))
 (segment (start 137.795 155.575) (end 119.38 155.575) (width 0.25) (layer F.Cu) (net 2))
 (segment (start 96.52 155.575) (end 95.885 154.94) (width 0.25) (layer B.Cu) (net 2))
 (segment (start 97.155 155.575) (end 96.52 155.575) (width 0.25) (layer B.Cu) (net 2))
 (segment (start 94.825 135.255) (end 95.885 135.255) (width 0.25) (layer B.Cu) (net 2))
 (segment (start 140.97 110.49) (end 116.84 110.49) (width 0.25) (layer F.Cu) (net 19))
 (segment (start 105.41 99.06) (end 99.06 99.06) (width 0.25) (layer F.Cu) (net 19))
 (segment (start 116.84 110.49) (end 105.41 99.06) (width 0.25) (layer F.Cu) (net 19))
 (segment (start 140.97 113.03) (end 116.84 113.03) (width 0.25) (layer F.Cu) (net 18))
 (segment (start 116.84 113.03) (end 105.41 101.6) (width 0.25) (layer F.Cu) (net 18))
 (segment (start 105.41 101.6) (end 99.06 101.6) (width 0.25) (layer F.Cu) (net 18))
 (via (at 95.25 115.57) (size 0.8) (drill 0.4) (layers F.Cu B.Cu) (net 4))
 (segment (start 92.71 102.87) (end 91.44 104.14) (width 0.25) (layer B.Cu) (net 4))
 (segment (start 91.44 104.14) (end 91.44 111.76) (width 0.25) (layer B.Cu) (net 4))
 (segment (start 95.25 115.57) (end 91.44 111.76) (width 0.25) (layer B.Cu) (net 4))
 (segment (start 95.25 115.57) (end 97.155 117.475) (width 0.25) (layer F.Cu) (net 4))
 (segment (start 99.06 106.68) (end 107.95 106.68) (width 0.25) (layer F.Cu) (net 17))
 (segment (start 116.84 115.57) (end 140.97 115.57) (width 0.25) (layer F.Cu) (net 17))
 (segment (start 107.95 106.68) (end 116.84 115.57) (width 0.25) (layer F.Cu) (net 17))
 (segment (start 92.71 100.33) (end 91.44 99.06) (width 0.25) (layer B.Cu) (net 10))
 (segment (start 91.44 99.06) (end 91.44 89.535) (width 0.25) (layer B.Cu) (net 10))
 (segment (start 141.03104 118.17104) (end 140.97 118.11) (width 0.25) (layer F.Cu) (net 12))
 (segment (start 140.97 118.11) (end 116.84 118.11) (width 0.25) (layer B.Cu) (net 12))
 (segment (start 106.49 128.46) (end 97.79 128.46) (width 0.25) (layer B.Cu) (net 12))
 (segment (start 116.84 118.11) (end 106.49 128.46) (width 0.25) (layer B.Cu) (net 12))
 (segment (start 97.79 130.46) (end 108.935 130.46) (width 0.25) (layer B.Cu) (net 11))
 (segment (start 118.745 120.65) (end 140.97 120.65) (width 0.25) (layer B.Cu) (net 11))
 (segment (start 108.935 130.46) (end 118.745 120.65) (width 0.25) (layer B.Cu) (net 11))
 (segment (start 92.075 157.48) (end 106.68 157.48) (width 0.25) (layer B.Cu) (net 15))
 (segment (start 140.97 123.19) (end 129.54 123.19) (width 0.25) (layer B.Cu) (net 15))
 (segment (start 129.54 123.19) (end 121.92 130.81) (width 0.25) (layer B.Cu) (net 15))
 (segment (start 121.92 130.81) (end 121.92 149.86) (width 0.25) (layer B.Cu) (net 15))
 (segment (start 114.3 157.48) (end 106.68 157.48) (width 0.25) (layer B.Cu) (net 15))
 (segment (start 121.92 149.86) (end 114.3 157.48) (width 0.25) (layer B.Cu) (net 15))
 (segment (start 92.075 141.605) (end 92.075 147.32) (width 0.25) (layer F.Cu) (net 8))
 (segment (start 93.345 66.675) (end 92.71 67.31) (width 0.25) (layer F.Cu) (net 7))
 (segment (start 98.425 66.675) (end 93.345 66.675) (width 0.25) (layer F.Cu) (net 7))
 (segment (start 138.43 140.335) (end 141.605 137.16) (width 0.25) (layer F.Cu) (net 9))
 (segment (start 141.605 137.16) (end 141.605 140.335) (width 0.25) (layer F.Cu) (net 9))
 (segment (start 137.16 140.335) (end 138.43 140.335) (width 0.25) (layer F.Cu) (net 9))
 (segment (start 141.605 134.62) (end 141.605 137.16) (width 0.25) (layer F.Cu) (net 9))
 (via (at 95.25 86.36) (size 0.8) (drill 0.4) (layers F.Cu B.Cu) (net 6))
 (segment (start 98.425 86.36) (end 95.25 86.36) (width 0.25) (layer F.Cu) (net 6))
 (segment (start 93.98 86.36) (end 92.71 85.09) (width 0.25) (layer B.Cu) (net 6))
 (segment (start 95.25 86.36) (end 93.98 86.36) (width 0.25) (layer B.Cu) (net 6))
 (segment (start 98.425 86.36) (end 101.6 89.535) (width 0.25) (layer F.Cu) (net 6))
 (segment (start 93.98 102.87) (end 95.25 104.14) (width 0.25) (layer F.Cu) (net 3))
 (segment (start 95.25 76.2) (end 97.79 73.66) (width 0.25) (layer F.Cu) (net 3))
 (segment (start 95.25 104.14) (end 99.06 104.14) (width 0.25) (layer F.Cu) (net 3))
 (segment (start 95.98 126.46) (end 95.25 125.73) (width 0.25) (layer F.Cu) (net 3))
 (segment (start 97.79 126.46) (end 95.98 126.46) (width 0.25) (layer F.Cu) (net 3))
 (segment (start 97.79 149.255002) (end 97.79 149.32) (width 0.25) (layer F.Cu) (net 3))
 (segment (start 95.25 146.715002) (end 97.79 149.255002) (width 0.25) (layer F.Cu) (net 3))
 (segment (start 95.25 125.73) (end 93.98 124.46) (width 0.25) (layer F.Cu) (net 3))
 (segment (start 93.98 102.87) (end 93.98 77.47) (width 0.25) (layer F.Cu) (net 3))
 (segment (start 93.98 77.47) (end 95.25 76.2) (width 0.25) (layer F.Cu) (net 3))
 (segment (start 133.56 140.335) (end 131.445 140.335) (width 0.25) (layer F.Cu) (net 3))
 (segment (start 95.25 125.73) (end 95.25 140.335) (width 0.25) (layer F.Cu) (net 3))
 (segment (start 94.19 121.075) (end 93.98 121.285) (width 0.25) (layer F.Cu) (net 3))
 (segment (start 97.155 121.075) (end 94.19 121.075) (width 0.25) (layer F.Cu) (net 3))
 (segment (start 93.98 121.285) (end 93.98 102.87) (width 0.25) (layer F.Cu) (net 3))
 (segment (start 93.98 124.46) (end 93.98 121.285) (width 0.25) (layer F.Cu) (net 3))
 (segment (start 133.56 140.335) (end 95.885 140.335) (width 0.25) (layer F.Cu) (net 3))
 (segment (start 95.25 140.97) (end 95.25 146.715002) (width 0.25) (layer F.Cu) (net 3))
 (segment (start 95.885 140.335) (end 95.25 140.97) (width 0.25) (layer F.Cu) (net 3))
 (segment (start 95.25 140.335) (end 95.25 140.97) (width 0.25) (layer F.Cu) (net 3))
 (segment (start 136.525 150.495) (end 135.89 149.86) (width 0.25) (layer F.Cu) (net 5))
 (segment (start 141.605 150.495) (end 136.525 150.495) (width 0.25) (layer F.Cu) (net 5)))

